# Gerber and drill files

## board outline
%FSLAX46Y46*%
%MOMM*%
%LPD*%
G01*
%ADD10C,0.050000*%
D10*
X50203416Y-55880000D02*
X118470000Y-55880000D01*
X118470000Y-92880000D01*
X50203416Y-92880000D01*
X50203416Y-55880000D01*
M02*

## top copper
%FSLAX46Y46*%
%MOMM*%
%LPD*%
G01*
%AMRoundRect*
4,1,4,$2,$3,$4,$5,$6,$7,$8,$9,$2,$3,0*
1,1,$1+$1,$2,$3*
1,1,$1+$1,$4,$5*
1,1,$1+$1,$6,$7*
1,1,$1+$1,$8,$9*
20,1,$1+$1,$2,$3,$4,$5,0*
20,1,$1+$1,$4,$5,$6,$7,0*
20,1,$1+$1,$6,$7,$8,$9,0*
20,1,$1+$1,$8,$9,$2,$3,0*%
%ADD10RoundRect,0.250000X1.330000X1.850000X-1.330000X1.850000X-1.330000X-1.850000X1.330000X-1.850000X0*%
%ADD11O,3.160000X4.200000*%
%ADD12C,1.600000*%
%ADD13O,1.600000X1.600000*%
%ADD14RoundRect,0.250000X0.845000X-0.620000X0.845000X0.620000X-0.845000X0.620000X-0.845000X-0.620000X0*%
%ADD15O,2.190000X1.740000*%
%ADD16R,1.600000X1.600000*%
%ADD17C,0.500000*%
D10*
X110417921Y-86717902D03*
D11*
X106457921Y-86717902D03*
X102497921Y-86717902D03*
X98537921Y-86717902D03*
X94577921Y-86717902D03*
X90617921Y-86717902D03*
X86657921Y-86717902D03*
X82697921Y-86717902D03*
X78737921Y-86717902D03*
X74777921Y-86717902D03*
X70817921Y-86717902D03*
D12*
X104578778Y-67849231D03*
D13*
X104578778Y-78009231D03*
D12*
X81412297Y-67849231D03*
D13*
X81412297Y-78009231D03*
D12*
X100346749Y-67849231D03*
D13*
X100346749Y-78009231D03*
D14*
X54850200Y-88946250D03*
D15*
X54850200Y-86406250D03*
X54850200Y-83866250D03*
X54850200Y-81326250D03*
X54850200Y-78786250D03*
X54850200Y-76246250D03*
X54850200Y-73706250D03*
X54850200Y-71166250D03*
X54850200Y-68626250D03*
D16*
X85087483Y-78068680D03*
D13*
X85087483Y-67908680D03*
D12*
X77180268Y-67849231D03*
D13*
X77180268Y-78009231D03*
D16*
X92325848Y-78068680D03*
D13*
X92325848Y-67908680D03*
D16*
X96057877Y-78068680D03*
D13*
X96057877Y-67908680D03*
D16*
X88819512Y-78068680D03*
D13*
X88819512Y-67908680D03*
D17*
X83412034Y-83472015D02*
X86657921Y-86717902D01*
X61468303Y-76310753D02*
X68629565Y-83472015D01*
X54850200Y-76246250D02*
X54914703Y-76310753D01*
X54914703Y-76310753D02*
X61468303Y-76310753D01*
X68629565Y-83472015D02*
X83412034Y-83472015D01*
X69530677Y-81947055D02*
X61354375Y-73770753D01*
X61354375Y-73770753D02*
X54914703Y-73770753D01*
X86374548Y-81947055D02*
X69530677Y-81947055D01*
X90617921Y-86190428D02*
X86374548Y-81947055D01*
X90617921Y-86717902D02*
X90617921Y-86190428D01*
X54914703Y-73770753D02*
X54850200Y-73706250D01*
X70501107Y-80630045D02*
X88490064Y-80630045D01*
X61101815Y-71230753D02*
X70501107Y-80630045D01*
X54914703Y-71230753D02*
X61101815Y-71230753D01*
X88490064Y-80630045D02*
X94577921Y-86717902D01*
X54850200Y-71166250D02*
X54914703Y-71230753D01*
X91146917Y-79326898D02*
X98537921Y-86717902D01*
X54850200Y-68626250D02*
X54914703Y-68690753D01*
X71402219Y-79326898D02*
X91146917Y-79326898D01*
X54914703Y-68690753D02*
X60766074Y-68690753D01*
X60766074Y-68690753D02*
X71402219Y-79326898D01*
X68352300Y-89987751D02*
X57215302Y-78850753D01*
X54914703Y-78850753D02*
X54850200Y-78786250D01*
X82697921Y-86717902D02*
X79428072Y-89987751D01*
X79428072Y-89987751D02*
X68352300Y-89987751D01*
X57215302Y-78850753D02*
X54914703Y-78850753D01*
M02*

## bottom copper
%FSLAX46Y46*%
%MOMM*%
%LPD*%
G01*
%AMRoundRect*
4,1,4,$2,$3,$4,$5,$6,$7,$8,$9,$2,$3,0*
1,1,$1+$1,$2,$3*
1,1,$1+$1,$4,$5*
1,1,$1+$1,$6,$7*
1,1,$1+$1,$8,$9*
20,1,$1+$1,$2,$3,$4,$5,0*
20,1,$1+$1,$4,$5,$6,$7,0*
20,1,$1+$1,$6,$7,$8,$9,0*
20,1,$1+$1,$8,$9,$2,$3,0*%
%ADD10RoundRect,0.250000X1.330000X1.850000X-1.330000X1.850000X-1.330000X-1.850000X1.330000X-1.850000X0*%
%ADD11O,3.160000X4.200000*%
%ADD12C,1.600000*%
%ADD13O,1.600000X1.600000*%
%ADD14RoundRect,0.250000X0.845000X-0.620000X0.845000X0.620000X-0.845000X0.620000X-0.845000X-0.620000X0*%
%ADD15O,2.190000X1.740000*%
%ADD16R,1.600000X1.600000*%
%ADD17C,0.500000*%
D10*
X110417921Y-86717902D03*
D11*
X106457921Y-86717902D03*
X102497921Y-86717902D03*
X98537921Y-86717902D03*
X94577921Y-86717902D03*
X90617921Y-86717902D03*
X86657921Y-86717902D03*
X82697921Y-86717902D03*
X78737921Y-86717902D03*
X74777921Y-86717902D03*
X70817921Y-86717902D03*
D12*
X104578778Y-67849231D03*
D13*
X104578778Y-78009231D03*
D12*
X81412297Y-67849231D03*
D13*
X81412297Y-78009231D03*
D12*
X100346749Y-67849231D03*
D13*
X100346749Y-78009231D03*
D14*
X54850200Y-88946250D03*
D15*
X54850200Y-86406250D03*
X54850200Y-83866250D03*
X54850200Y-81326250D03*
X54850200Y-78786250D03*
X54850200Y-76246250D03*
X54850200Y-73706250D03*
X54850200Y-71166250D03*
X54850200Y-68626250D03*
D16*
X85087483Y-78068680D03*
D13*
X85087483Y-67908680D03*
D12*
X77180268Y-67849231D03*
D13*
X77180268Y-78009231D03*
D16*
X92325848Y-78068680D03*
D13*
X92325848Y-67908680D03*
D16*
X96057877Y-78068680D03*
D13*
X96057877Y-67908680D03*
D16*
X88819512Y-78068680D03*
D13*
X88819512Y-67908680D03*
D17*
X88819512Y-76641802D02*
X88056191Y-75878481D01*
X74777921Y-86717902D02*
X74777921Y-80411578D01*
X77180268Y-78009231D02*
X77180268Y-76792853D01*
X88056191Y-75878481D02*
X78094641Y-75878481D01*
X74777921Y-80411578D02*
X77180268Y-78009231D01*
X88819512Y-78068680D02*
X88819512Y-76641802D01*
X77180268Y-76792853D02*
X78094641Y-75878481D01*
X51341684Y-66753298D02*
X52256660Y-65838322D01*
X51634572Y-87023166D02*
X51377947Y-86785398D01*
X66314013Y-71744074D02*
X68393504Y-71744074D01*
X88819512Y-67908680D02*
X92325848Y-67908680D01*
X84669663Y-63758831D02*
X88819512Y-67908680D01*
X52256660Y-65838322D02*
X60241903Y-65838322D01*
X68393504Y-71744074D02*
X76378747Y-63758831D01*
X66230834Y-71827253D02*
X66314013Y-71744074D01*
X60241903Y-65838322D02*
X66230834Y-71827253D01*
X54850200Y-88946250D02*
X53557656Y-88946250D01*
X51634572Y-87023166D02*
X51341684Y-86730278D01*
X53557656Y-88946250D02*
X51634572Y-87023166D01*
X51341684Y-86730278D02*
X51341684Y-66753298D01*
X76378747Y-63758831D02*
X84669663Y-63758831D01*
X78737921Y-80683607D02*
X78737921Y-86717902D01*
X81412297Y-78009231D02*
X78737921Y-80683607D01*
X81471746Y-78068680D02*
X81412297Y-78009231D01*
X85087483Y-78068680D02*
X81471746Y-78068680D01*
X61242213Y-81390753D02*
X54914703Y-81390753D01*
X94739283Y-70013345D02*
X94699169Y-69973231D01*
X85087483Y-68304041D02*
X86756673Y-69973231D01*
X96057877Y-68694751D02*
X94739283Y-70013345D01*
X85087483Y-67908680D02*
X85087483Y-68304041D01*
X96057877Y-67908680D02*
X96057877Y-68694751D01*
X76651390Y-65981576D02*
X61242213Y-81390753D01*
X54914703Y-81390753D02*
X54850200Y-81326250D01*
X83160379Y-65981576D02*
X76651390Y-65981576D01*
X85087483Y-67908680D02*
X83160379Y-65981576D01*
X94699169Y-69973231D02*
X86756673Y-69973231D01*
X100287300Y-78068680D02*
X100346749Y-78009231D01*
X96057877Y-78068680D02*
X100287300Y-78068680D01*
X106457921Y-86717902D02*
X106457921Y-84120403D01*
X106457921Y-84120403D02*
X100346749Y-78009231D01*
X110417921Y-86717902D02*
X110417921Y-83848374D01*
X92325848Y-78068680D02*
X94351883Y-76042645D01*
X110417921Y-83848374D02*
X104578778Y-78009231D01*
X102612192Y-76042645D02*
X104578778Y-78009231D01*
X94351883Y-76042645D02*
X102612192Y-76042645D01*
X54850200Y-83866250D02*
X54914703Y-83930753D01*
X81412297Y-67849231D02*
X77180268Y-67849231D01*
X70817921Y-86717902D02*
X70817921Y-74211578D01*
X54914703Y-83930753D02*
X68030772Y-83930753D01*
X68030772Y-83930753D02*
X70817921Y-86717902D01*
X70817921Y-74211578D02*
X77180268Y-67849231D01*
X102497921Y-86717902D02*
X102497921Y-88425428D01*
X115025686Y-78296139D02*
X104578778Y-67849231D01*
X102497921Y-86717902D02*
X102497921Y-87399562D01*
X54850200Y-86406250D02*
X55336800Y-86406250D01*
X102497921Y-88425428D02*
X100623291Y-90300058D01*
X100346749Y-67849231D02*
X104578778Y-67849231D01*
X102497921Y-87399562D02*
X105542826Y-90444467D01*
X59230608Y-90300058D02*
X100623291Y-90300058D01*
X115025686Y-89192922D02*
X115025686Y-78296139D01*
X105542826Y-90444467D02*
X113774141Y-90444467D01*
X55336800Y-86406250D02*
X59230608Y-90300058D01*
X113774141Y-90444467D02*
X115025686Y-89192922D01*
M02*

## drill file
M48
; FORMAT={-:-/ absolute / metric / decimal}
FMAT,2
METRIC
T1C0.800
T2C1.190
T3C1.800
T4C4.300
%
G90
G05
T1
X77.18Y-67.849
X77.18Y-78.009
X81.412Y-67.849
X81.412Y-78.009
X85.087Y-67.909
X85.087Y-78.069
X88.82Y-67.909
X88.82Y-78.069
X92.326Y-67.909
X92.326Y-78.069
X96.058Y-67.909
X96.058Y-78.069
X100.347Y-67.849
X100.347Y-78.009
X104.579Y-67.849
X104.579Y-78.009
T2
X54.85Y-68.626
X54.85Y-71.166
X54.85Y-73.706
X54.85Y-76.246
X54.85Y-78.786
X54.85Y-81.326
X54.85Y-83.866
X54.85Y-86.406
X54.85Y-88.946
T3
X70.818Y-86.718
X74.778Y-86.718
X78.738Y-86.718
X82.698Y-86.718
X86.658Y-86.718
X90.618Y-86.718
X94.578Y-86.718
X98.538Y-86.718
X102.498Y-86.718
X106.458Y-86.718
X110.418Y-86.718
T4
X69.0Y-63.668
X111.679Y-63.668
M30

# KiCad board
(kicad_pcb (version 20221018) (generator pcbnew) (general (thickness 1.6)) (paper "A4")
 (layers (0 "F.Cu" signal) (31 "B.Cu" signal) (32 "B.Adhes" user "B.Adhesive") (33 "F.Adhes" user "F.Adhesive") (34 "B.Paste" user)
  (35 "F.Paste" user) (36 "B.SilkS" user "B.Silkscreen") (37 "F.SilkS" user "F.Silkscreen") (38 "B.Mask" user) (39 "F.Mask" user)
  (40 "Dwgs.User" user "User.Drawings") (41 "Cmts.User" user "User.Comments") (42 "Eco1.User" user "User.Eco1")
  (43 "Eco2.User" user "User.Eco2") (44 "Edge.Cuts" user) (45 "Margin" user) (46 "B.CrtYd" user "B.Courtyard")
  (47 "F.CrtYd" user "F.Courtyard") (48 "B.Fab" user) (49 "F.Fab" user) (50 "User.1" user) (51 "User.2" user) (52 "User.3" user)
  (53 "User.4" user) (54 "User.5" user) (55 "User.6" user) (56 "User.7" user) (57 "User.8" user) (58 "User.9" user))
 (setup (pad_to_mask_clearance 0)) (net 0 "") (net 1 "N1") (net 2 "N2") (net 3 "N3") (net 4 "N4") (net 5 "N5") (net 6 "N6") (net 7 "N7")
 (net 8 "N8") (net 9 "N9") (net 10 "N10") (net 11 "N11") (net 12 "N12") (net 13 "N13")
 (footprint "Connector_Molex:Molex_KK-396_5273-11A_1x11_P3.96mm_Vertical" (layer "F.Cu") (at 110.417921 86.717902 180)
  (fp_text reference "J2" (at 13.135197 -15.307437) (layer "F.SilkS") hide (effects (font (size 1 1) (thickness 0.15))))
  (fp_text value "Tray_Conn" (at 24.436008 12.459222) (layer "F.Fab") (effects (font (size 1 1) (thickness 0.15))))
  (pad "1" thru_hole roundrect (at 0 0 180) (size 3.16 4.2) (drill 1.8) (layers "*.Cu" "*.Mask") (roundrect_rratio 0.07911392405)
   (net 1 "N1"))
  (pad "2" thru_hole oval (at 3.96 0 180) (size 3.16 4.2) (drill 1.8) (layers "*.Cu" "*.Mask") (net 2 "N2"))
  (pad "3" thru_hole oval (at 7.92 0 180) (size 3.16 4.2) (drill 1.8) (layers "*.Cu" "*.Mask") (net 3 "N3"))
  (pad "4" thru_hole oval (at 11.88 0 180) (size 3.16 4.2) (drill 1.8) (layers "*.Cu" "*.Mask") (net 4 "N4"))
  (pad "5" thru_hole oval (at 15.84 0 180) (size 3.16 4.2) (drill 1.8) (layers "*.Cu" "*.Mask") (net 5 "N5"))
  (pad "6" thru_hole oval (at 19.8 0 180) (size 3.16 4.2) (drill 1.8) (layers "*.Cu" "*.Mask") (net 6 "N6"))
  (pad "7" thru_hole oval (at 23.76 0 180) (size 3.16 4.2) (drill 1.8) (layers "*.Cu" "*.Mask") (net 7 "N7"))
  (pad "8" thru_hole oval (at 27.72 0 180) (size 3.16 4.2) (drill 1.8) (layers "*.Cu" "*.Mask") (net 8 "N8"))
  (pad "9" thru_hole oval (at 31.68 0 180) (size 3.16 4.2) (drill 1.8) (layers "*.Cu" "*.Mask") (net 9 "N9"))
  (pad "10" thru_hole oval (at 35.64 0 180) (size 3.16 4.2) (drill 1.8) (layers "*.Cu" "*.Mask") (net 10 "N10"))
  (pad "11" thru_hole oval (at 39.6 0 180) (size 3.16 4.2) (drill 1.8) (layers "*.Cu" "*.Mask") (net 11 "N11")))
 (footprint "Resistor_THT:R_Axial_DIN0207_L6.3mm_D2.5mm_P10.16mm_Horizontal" (layer "F.Cu") (at 104.578778 67.849231 -90)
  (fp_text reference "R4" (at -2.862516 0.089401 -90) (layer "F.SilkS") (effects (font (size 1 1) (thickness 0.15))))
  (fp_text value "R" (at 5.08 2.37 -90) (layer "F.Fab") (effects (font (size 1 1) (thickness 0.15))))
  (pad "1" thru_hole circle (at 0 0 270) (size 1.6 1.6) (drill 0.8) (layers "*.Cu" "*.Mask") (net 3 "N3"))
  (pad "2" thru_hole oval (at 10.16 0 270) (size 1.6 1.6) (drill 0.8) (layers "*.Cu" "*.Mask") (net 1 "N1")))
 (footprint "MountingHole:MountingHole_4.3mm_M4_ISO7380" (layer "F.Cu") (at 69 63.667921)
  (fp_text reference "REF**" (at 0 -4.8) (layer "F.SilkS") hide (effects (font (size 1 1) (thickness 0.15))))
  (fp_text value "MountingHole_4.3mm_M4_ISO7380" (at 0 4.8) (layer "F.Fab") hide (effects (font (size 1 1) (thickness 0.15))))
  (pad "" np_thru_hole circle (at 0 0) (size 4.3 4.3) (drill 4.3) (layers "*.Cu" "*.Mask")))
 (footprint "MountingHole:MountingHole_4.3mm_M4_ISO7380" (layer "F.Cu") (at 111.679187 63.667921)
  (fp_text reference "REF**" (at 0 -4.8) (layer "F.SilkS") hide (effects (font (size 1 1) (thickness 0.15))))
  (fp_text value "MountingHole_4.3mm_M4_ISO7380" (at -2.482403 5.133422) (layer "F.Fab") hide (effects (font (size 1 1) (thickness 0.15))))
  (pad "" np_thru_hole circle (at 0 0) (size 4.3 4.3) (drill 4.3) (layers "*.Cu" "*.Mask")))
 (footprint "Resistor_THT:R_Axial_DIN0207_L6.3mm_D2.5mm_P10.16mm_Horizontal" (layer "F.Cu") (at 81.412297 67.849231 -90)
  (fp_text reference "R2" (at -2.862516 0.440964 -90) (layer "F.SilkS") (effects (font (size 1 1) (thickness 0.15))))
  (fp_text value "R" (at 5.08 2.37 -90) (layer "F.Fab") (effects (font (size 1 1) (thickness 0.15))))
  (pad "1" thru_hole circle (at 0 0 270) (size 1.6 1.6) (drill 0.8) (layers "*.Cu" "*.Mask") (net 11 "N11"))
  (pad "2" thru_hole oval (at 10.16 0 270) (size 1.6 1.6) (drill 0.8) (layers "*.Cu" "*.Mask") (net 9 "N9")))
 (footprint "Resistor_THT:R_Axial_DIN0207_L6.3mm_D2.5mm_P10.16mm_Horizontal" (layer "F.Cu") (at 100.346749 67.849231 -90)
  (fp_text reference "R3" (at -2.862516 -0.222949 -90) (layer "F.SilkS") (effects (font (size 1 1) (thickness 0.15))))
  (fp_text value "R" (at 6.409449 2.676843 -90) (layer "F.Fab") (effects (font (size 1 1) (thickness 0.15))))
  (pad "1" thru_hole circle (at 0 0 270) (size 1.6 1.6) (drill 0.8) (layers "*.Cu" "*.Mask") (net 3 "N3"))
  (pad "2" thru_hole oval (at 10.16 0 270) (size 1.6 1.6) (drill 0.8) (layers "*.Cu" "*.Mask") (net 2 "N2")))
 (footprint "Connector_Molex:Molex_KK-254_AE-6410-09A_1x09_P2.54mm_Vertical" (layer "F.Cu") (at 54.8502 88.94625 90)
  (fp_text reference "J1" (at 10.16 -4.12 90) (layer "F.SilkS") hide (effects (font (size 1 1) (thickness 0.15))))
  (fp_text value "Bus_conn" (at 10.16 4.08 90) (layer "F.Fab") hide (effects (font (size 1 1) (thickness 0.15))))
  (pad "1" thru_hole roundrect (at 0 0 90) (size 1.74 2.19) (drill 1.19) (layers "*.Cu" "*.Mask") (roundrect_rratio 0.1436781609)
   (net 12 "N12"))
  (pad "2" thru_hole oval (at 2.54 0 90) (size 1.74 2.19) (drill 1.19) (layers "*.Cu" "*.Mask") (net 3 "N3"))
  (pad "3" thru_hole oval (at 5.08 0 90) (size 1.74 2.19) (drill 1.19) (layers "*.Cu" "*.Mask") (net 11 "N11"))
  (pad "4" thru_hole oval (at 7.62 0 90) (size 1.74 2.19) (drill 1.19) (layers "*.Cu" "*.Mask") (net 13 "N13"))
  (pad "5" thru_hole oval (at 10.16 0 90) (size 1.74 2.19) (drill 1.19) (layers "*.Cu" "*.Mask") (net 8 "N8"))
  (pad "6" thru_hole oval (at 12.7 0 90) (size 1.74 2.19) (drill 1.19) (layers "*.Cu" "*.Mask") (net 7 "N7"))
  (pad "7" thru_hole oval (at 15.24 0 90) (size 1.74 2.19) (drill 1.19) (layers "*.Cu" "*.Mask") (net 6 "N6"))
  (pad "8" thru_hole oval (at 17.78 0 90) (size 1.74 2.19) (drill 1.19) (layers "*.Cu" "*.Mask") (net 5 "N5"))
  (pad "9" thru_hole oval (at 20.32 0 90) (size 1.74 2.19) (drill 1.19) (layers "*.Cu" "*.Mask") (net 4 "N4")))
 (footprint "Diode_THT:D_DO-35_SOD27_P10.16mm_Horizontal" (layer "F.Cu") (at 85.087483 78.06868 90)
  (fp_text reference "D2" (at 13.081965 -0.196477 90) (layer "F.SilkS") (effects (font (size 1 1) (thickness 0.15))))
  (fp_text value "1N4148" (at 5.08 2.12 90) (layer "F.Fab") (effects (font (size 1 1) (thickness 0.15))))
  (pad "1" thru_hole rect (at 0 0 90) (size 1.6 1.6) (drill 0.8) (layers "*.Cu" "*.Mask") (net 9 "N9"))
  (pad "2" thru_hole oval (at 10.16 0 90) (size 1.6 1.6) (drill 0.8) (layers "*.Cu" "*.Mask") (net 13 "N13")))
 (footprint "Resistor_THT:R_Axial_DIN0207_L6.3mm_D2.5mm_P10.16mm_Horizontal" (layer "F.Cu") (at 77.180268 67.849231 -90)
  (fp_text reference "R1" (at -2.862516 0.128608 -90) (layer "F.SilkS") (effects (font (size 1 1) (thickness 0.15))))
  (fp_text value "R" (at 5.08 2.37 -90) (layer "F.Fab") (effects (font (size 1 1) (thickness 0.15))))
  (pad "1" thru_hole circle (at 0 0 270) (size 1.6 1.6) (drill 0.8) (layers "*.Cu" "*.Mask") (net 11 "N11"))
  (pad "2" thru_hole oval (at 10.16 0 270) (size 1.6 1.6) (drill 0.8) (layers "*.Cu" "*.Mask") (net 10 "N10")))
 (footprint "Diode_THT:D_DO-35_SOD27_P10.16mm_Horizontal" (layer "F.Cu") (at 92.325848 78.06868 90)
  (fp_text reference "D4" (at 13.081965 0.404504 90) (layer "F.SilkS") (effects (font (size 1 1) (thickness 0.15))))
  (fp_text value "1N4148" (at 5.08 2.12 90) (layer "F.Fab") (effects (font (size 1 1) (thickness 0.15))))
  (pad "1" thru_hole rect (at 0 0 90) (size 1.6 1.6) (drill 0.8) (layers "*.Cu" "*.Mask") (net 1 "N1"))
  (pad "2" thru_hole oval (at 10.16 0 90) (size 1.6 1.6) (drill 0.8) (layers "*.Cu" "*.Mask") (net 12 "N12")))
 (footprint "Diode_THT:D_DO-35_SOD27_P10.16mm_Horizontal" (layer "F.Cu") (at 96.057877 78.06868 90)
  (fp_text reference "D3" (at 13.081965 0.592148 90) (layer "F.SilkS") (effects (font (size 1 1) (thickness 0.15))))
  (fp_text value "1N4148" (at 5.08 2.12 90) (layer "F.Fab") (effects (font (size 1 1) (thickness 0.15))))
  (pad "1" thru_hole rect (at 0 0 90) (size 1.6 1.6) (drill 0.8) (layers "*.Cu" "*.Mask") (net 2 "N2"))
  (pad "2" thru_hole oval (at 10.16 0 90) (size 1.6 1.6) (drill 0.8) (layers "*.Cu" "*.Mask") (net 13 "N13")))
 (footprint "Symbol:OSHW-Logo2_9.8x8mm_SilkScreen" (layer "F.Cu") (at 56.81449 60.716683)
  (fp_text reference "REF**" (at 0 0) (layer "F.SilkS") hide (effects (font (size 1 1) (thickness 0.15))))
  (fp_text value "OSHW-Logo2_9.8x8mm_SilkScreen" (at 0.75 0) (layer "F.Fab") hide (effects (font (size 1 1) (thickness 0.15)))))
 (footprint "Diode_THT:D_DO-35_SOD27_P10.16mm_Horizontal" (layer "F.Cu") (at 88.819512 78.06868 90)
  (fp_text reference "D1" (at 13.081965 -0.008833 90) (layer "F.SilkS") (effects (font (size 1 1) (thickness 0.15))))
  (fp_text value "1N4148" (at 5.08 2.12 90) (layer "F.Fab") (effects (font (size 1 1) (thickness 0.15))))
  (pad "1" thru_hole rect (at 0 0 90) (size 1.6 1.6) (drill 0.8) (layers "*.Cu" "*.Mask") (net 10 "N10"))
  (pad "2" thru_hole oval (at 10.16 0 90) (size 1.6 1.6) (drill 0.8) (layers "*.Cu" "*.Mask") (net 12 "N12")))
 (gr_rect (start 50.203416 55.88) (end 118.47 92.88) (stroke (width 0.05) (type default)) (fill none) (layer "Edge.Cuts"))
 (segment (start 88.819512 76.641802) (end 88.056191 75.878481) (width 0.5) (layer "B.Cu") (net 10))
 (segment (start 74.777921 86.717902) (end 74.777921 80.411578) (width 0.5) (layer "B.Cu") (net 10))
 (segment (start 77.180268 78.009231) (end 77.180268 76.792853) (width 0.5) (layer "B.Cu") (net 10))
 (segment (start 88.056191 75.878481) (end 78.094641 75.878481) (width 0.5) (layer "B.Cu") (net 10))
 (segment (start 74.777921 80.411578) (end 77.180268 78.009231) (width 0.5) (layer "B.Cu") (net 10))
 (segment (start 88.819512 78.06868) (end 88.819512 76.641802) (width 0.5) (layer "B.Cu") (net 10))
 (segment (start 77.180268 76.792853) (end 78.094641 75.878481) (width 0.5) (layer "B.Cu") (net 10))
 (segment (start 51.341684 66.753298) (end 52.25666 65.838322) (width 0.5) (layer "B.Cu") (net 12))
 (segment (start 51.634572 87.023166) (end 51.377947 86.785398) (width 0.5) (layer "B.Cu") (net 12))
 (segment (start 66.314013 71.744074) (end 68.393504 71.744074) (width 0.5) (layer "B.Cu") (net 12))
 (segment (start 88.819512 67.90868) (end 92.325848 67.90868) (width 0.5) (layer "B.Cu") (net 12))
 (segment (start 84.669663 63.758831) (end 88.819512 67.90868) (width 0.5) (layer "B.Cu") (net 12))
 (segment (start 52.25666 65.838322) (end 60.241903 65.838322) (width 0.5) (layer "B.Cu") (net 12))
 (segment (start 68.393504 71.744074) (end 76.378747 63.758831) (width 0.5) (layer "B.Cu") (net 12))
 (segment (start 66.230834 71.827253) (end 66.314013 71.744074) (width 0.5) (layer "B.Cu") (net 12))
 (segment (start 60.241903 65.838322) (end 66.230834 71.827253) (width 0.5) (layer "B.Cu") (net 12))
 (segment (start 54.8502 88.94625) (end 53.557656 88.94625) (width 0.5) (layer "B.Cu") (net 12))
 (segment (start 51.634572 87.023166) (end 51.341684 86.730278) (width 0.5) (layer "B.Cu") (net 12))
 (segment (start 53.557656 88.94625) (end 51.634572 87.023166) (width 0.5) (layer "B.Cu") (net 12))
 (segment (start 51.341684 86.730278) (end 51.341684 66.753298) (width 0.5) (layer "B.Cu") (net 12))
 (segment (start 76.378747 63.758831) (end 84.669663 63.758831) (width 0.5) (layer "B.Cu") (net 12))
 (segment (start 78.737921 80.683607) (end 78.737921 86.717902) (width 0.5) (layer "B.Cu") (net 9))
 (segment (start 81.412297 78.009231) (end 78.737921 80.683607) (width 0.5) (layer "B.Cu") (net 9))
 (segment (start 81.471746 78.06868) (end 81.412297 78.009231) (width 0.5) (layer "B.Cu") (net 9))
 (segment (start 85.087483 78.06868) (end 81.471746 78.06868) (width 0.5) (layer "B.Cu") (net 9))
 (segment (start 61.242213 81.390753) (end 54.914703 81.390753) (width 0.5) (layer "B.Cu") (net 13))
 (segment (start 94.739283 70.013345) (end 94.699169 69.973231) (width 0.5) (layer "B.Cu") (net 13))
 (segment (start 85.087483 68.304041) (end 86.756673 69.973231) (width 0.5) (layer "B.Cu") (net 13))
 (segment (start 96.057877 68.694751) (end 94.739283 70.013345) (width 0.5) (layer "B.Cu") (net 13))
 (segment (start 85.087483 67.90868) (end 85.087483 68.304041) (width 0.5) (layer "B.Cu") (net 13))
 (segment (start 96.057877 67.90868) (end 96.057877 68.694751) (width 0.5) (layer "B.Cu") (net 13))
 (segment (start 76.65139 65.981576) (end 61.242213 81.390753) (width 0.5) (layer "B.Cu") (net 13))
 (segment (start 54.914703 81.390753) (end 54.8502 81.32625) (width 0.5) (layer "B.Cu") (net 13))
 (segment (start 83.160379 65.981576) (end 76.65139 65.981576) (width 0.5) (layer "B.Cu") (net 13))
 (segment (start 85.087483 67.90868) (end 83.160379 65.981576) (width 0.5) (layer "B.Cu") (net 13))
 (segment (start 94.699169 69.973231) (end 86.756673 69.973231) (width 0.5) (layer "B.Cu") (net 13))
 (segment (start 100.2873 78.06868) (end 100.346749 78.009231) (width 0.5) (layer "B.Cu") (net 2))
 (segment (start 96.057877 78.06868) (end 100.2873 78.06868) (width 0.5) (layer "B.Cu") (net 2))
 (segment (start 106.457921 86.717902) (end 106.457921 84.120403) (width 0.5) (layer "B.Cu") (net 2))
 (segment (start 106.457921 84.120403) (end 100.346749 78.009231) (width 0.5) (layer "B.Cu") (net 2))
 (segment (start 110.417921 86.717902) (end 110.417921 83.848374) (width 0.5) (layer "B.Cu") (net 1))
 (segment (start 92.325848 78.06868) (end 94.351883 76.042645) (width 0.5) (layer "B.Cu") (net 1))
 (segment (start 110.417921 83.848374) (end 104.578778 78.009231) (width 0.5) (layer "B.Cu") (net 1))
 (segment (start 102.612192 76.042645) (end 104.578778 78.009231) (width 0.5) (layer "B.Cu") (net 1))
 (segment (start 94.351883 76.042645) (end 102.612192 76.042645) (width 0.5) (layer "B.Cu") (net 1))
 (segment (start 54.8502 83.86625) (end 54.914703 83.930753) (width 0.5) (layer "B.Cu") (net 11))
 (segment (start 81.412297 67.849231) (end 77.180268 67.849231) (width 0.5) (layer "B.Cu") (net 11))
 (segment (start 70.817921 86.717902) (end 70.817921 74.211578) (width 0.5) (layer "B.Cu") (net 11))
 (segment (start 54.914703 83.930753) (end 68.030772 83.930753) (width 0.5) (layer "B.Cu") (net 11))
 (segment (start 68.030772 83.930753) (end 70.817921 86.717902) (width 0.5) (layer "B.Cu") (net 11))
 (segment (start 70.817921 74.211578) (end 77.180268 67.849231) (width 0.5) (layer "B.Cu") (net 11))
 (segment (start 102.497921 86.717902) (end 102.497921 88.425428) (width 0.5) (layer "B.Cu") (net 3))
 (segment (start 115.025686 78.296139) (end 104.578778 67.849231) (width 0.5) (layer "B.Cu") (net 3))
 (segment (start 102.497921 86.717902) (end 102.497921 87.399562) (width 0.5) (layer "B.Cu") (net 3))
 (segment (start 54.8502 86.40625) (end 55.3368 86.40625) (width 0.5) (layer "B.Cu") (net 3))
 (segment (start 102.497921 88.425428) (end 100.623291 90.300058) (width 0.5) (layer "B.Cu") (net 3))
 (segment (start 100.346749 67.849231) (end 104.578778 67.849231) (width 0.5) (layer "B.Cu") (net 3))
 (segment (start 102.497921 87.399562) (end 105.542826 90.444467) (width 0.5) (layer "B.Cu") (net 3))
 (segment (start 59.230608 90.300058) (end 100.623291 90.300058) (width 0.5) (layer "B.Cu") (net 3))
 (segment (start 115.025686 89.192922) (end 115.025686 78.296139) (width 0.5) (layer "B.Cu") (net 3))
 (segment (start 105.542826 90.444467) (end 113.774141 90.444467) (width 0.5) (layer "B.Cu") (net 3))
 (segment (start 55.3368 86.40625) (end 59.230608 90.300058) (width 0.5) (layer "B.Cu") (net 3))
 (segment (start 113.774141 90.444467) (end 115.025686 89.192922) (width 0.5) (layer "B.Cu") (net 3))
 (segment (start 83.412034 83.472015) (end 86.657921 86.717902) (width 0.5) (layer "F.Cu") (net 7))
 (segment (start 61.468303 76.310753) (end 68.629565 83.472015) (width 0.5) (layer "F.Cu") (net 7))
 (segment (start 54.8502 76.24625) (end 54.914703 76.310753) (width 0.5) (layer "F.Cu") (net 7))
 (segment (start 54.914703 76.310753) (end 61.468303 76.310753) (width 0.5) (layer "F.Cu") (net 7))
 (segment (start 68.629565 83.472015) (end 83.412034 83.472015) (width 0.5) (layer "F.Cu") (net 7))
 (segment (start 69.530677 81.947055) (end 61.354375 73.770753) (width 0.5) (layer "F.Cu") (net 6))
 (segment (start 61.354375 73.770753) (end 54.914703 73.770753) (width 0.5) (layer "F.Cu") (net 6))
 (segment (start 86.374548 81.947055) (end 69.530677 81.947055) (width 0.5) (layer "F.Cu") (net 6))
 (segment (start 90.617921 86.190428) (end 86.374548 81.947055) (width 0.5) (layer "F.Cu") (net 6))
 (segment (start 90.617921 86.717902) (end 90.617921 86.190428) (width 0.5) (layer "F.Cu") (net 6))
 (segment (start 54.914703 73.770753) (end 54.8502 73.70625) (width 0.5) (layer "F.Cu") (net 6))
 (segment (start 70.501107 80.630045) (end 88.490064 80.630045) (width 0.5) (layer "F.Cu") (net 5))
 (segment (start 61.101815 71.230753) (end 70.501107 80.630045) (width 0.5) (layer "F.Cu") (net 5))
 (segment (start 54.914703 71.230753) (end 61.101815 71.230753) (width 0.5) (layer "F.Cu") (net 5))
 (segment (start 88.490064 80.630045) (end 94.577921 86.717902) (width 0.5) (layer "F.Cu") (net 5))
 (segment (start 54.8502 71.16625) (end 54.914703 71.230753) (width 0.5) (layer "F.Cu") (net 5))
 (segment (start 91.146917 79.326898) (end 98.537921 86.717902) (width 0.5) (layer "F.Cu") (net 4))
 (segment (start 54.8502 68.62625) (end 54.914703 68.690753) (width 0.5) (layer "F.Cu") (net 4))
 (segment (start 71.402219 79.326898) (end 91.146917 79.326898) (width 0.5) (layer "F.Cu") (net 4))
 (segment (start 54.914703 68.690753) (end 60.766074 68.690753) (width 0.5) (layer "F.Cu") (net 4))
 (segment (start 60.766074 68.690753) (end 71.402219 79.326898) (width 0.5) (layer "F.Cu") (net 4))
 (segment (start 68.3523 89.987751) (end 57.215302 78.850753) (width 0.5) (layer "F.Cu") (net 8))
 (segment (start 54.914703 78.850753) (end 54.8502 78.78625) (width 0.5) (layer "F.Cu") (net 8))
 (segment (start 82.697921 86.717902) (end 79.428072 89.987751) (width 0.5) (layer "F.Cu") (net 8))
 (segment (start 79.428072 89.987751) (end 68.3523 89.987751) (width 0.5) (layer "F.Cu") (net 8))
 (segment (start 57.215302 78.850753) (end 54.914703 78.850753) (width 0.5) (layer "F.Cu") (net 8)))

